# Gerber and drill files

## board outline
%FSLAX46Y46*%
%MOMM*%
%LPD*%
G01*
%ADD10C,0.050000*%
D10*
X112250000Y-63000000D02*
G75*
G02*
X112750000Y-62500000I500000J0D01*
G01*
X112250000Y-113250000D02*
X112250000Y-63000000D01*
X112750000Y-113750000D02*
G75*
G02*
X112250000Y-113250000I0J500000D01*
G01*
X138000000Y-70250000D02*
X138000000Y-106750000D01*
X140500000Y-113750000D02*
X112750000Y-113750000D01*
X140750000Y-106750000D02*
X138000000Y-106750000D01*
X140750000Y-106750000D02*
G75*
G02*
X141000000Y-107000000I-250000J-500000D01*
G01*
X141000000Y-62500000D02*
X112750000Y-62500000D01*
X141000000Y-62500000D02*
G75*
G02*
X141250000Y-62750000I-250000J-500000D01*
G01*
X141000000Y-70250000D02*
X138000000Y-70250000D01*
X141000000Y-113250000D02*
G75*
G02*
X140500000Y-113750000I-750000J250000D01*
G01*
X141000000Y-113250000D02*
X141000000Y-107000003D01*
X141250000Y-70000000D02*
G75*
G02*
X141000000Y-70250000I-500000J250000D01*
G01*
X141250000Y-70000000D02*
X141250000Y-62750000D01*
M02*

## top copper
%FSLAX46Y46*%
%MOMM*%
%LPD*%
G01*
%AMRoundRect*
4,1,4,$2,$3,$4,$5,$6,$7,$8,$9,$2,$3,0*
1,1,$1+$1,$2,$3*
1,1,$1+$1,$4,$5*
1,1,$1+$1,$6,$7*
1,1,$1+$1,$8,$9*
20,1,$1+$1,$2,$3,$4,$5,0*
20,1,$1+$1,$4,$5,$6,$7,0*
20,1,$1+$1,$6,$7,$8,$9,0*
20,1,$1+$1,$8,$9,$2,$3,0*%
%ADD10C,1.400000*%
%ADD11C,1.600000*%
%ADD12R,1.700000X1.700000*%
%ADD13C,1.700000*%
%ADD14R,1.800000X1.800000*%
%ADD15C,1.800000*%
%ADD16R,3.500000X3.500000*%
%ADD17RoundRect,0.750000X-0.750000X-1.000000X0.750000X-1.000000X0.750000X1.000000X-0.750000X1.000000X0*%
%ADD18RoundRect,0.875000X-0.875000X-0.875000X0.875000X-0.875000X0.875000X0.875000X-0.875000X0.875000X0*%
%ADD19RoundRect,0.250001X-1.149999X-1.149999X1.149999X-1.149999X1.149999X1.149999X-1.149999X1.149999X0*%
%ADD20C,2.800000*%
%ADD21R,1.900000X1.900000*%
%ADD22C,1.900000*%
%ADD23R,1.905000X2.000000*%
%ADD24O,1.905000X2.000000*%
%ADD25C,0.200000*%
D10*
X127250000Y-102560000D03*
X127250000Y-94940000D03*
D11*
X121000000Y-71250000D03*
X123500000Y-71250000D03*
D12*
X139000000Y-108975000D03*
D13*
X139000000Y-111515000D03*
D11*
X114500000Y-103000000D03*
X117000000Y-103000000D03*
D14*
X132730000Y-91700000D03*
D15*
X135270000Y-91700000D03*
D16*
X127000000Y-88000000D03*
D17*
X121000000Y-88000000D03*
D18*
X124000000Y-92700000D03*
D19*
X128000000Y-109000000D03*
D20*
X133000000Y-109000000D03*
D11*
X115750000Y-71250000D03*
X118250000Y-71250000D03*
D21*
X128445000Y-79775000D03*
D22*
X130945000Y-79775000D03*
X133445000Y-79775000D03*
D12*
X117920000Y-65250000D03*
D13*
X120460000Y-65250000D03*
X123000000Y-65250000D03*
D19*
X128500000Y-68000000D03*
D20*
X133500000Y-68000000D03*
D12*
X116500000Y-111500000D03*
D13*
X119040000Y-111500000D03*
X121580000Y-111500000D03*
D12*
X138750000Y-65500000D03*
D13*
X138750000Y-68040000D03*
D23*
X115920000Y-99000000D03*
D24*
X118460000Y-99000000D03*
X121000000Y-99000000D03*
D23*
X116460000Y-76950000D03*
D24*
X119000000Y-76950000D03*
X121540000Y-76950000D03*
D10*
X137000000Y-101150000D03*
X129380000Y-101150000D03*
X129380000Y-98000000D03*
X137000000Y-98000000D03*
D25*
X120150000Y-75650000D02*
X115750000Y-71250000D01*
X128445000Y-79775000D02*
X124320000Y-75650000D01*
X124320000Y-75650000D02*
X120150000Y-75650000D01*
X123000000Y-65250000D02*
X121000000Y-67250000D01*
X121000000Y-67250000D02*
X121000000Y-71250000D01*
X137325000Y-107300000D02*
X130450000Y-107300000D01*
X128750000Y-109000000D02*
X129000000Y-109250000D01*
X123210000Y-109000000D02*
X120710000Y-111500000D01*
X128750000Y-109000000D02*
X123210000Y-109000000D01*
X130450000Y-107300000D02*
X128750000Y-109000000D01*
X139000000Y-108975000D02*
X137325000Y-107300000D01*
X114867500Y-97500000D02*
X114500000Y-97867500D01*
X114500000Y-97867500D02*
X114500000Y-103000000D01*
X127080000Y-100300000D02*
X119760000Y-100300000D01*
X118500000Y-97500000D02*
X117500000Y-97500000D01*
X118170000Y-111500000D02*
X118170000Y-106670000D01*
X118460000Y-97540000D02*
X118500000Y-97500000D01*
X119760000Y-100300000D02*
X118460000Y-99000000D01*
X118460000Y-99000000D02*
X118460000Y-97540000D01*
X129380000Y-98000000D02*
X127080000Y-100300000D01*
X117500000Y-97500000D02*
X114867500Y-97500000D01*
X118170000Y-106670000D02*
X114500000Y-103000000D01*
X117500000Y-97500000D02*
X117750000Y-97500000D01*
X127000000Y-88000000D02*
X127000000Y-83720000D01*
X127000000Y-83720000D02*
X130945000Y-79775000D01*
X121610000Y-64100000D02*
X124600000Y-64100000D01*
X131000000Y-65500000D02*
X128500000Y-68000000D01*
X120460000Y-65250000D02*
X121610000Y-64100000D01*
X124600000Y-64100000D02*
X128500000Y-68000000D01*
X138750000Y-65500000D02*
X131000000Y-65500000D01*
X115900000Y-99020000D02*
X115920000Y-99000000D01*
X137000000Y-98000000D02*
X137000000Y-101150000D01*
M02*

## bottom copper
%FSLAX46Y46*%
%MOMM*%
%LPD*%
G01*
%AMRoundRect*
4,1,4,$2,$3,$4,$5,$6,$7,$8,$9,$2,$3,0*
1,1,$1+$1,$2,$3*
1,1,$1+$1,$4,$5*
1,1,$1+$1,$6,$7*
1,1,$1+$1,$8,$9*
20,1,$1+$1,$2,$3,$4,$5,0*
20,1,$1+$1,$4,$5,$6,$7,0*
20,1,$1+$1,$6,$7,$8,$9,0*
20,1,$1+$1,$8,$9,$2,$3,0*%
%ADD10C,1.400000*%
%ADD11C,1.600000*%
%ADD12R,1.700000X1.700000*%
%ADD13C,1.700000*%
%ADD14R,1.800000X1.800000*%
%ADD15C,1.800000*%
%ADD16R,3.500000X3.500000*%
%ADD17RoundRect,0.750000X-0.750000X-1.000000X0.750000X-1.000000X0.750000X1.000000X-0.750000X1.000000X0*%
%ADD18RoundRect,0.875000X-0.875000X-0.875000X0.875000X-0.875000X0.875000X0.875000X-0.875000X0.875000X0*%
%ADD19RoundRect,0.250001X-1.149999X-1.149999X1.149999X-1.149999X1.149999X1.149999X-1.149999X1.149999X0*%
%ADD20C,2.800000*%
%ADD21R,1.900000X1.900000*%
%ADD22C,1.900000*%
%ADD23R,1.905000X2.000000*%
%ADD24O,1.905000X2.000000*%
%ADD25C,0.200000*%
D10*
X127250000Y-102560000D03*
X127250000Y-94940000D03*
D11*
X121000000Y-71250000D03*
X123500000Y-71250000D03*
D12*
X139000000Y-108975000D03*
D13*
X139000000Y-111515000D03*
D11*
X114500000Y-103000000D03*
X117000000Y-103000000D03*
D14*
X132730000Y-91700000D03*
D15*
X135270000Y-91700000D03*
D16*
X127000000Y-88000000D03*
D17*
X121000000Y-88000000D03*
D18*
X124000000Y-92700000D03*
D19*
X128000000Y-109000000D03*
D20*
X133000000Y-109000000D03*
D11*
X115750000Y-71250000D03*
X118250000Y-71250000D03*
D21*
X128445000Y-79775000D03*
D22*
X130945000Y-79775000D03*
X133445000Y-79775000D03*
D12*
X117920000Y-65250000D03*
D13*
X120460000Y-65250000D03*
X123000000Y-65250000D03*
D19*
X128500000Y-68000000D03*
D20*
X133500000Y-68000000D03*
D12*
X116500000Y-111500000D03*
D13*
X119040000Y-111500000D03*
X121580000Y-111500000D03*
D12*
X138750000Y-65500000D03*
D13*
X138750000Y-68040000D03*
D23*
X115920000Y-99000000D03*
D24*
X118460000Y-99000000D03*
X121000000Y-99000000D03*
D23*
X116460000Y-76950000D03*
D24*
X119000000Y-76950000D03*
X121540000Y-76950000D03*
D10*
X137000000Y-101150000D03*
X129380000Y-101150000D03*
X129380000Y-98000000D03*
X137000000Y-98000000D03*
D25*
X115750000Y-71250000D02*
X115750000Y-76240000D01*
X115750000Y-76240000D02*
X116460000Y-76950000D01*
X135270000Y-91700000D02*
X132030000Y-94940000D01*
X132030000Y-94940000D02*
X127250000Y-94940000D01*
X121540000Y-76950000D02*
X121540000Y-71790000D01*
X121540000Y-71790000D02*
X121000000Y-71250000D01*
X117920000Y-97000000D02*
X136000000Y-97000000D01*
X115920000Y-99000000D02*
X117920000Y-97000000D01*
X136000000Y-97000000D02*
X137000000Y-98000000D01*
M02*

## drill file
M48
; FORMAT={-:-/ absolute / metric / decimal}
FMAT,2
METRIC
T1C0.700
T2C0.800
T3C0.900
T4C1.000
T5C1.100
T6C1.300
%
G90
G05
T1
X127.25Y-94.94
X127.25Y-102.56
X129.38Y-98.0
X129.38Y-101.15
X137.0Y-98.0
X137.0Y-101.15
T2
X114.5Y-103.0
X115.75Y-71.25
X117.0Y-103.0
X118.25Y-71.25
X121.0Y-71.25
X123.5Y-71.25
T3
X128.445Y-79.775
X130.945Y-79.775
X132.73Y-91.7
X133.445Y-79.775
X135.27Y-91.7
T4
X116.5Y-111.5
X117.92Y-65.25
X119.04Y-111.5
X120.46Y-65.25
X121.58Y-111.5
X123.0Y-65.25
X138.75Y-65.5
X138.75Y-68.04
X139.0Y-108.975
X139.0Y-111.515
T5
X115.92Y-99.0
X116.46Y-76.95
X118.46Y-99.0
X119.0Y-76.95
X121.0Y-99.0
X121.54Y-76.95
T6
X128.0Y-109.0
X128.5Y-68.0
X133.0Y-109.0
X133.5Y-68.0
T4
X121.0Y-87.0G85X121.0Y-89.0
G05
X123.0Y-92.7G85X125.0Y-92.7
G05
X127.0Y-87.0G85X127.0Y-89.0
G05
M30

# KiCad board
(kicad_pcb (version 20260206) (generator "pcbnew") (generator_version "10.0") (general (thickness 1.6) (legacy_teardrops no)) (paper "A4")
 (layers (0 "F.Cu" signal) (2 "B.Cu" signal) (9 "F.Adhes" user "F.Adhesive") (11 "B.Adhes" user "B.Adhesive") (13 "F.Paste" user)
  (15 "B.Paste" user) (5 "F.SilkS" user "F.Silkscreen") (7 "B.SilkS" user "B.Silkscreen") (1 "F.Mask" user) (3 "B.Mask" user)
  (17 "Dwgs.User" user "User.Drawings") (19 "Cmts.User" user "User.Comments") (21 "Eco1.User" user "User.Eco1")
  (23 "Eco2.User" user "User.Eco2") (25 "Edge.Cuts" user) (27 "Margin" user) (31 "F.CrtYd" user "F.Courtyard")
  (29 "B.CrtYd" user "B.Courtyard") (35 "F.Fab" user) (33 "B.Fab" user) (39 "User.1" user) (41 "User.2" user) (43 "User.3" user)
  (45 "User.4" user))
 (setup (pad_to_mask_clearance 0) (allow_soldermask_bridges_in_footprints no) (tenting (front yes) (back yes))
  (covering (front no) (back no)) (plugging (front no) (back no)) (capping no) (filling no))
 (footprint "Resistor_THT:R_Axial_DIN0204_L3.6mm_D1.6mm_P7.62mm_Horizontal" (layer "F.Cu") (at 127.25 102.56 90)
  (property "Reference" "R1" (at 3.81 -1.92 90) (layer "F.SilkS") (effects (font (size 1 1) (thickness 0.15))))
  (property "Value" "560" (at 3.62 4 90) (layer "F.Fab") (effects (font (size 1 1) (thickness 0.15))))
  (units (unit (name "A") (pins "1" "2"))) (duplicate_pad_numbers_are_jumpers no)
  (pad "1" thru_hole circle (at 0 0 90) (size 1.4 1.4) (drill 0.7) (layers "*.Cu" "*.Mask") (remove_unused_layers no) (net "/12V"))
  (pad "2" thru_hole circle (at 7.62 0 90) (size 1.4 1.4) (drill 0.7) (layers "*.Cu" "*.Mask") (remove_unused_layers no) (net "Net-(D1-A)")))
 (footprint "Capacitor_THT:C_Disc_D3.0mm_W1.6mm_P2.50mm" (layer "F.Cu") (at 121 71.25)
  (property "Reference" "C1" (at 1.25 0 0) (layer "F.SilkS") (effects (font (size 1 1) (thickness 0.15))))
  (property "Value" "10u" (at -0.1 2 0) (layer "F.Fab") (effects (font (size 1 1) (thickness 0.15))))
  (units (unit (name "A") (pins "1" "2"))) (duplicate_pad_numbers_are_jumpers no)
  (pad "1" thru_hole circle (at 0 0) (size 1.6 1.6) (drill 0.8) (layers "*.Cu" "*.Mask") (remove_unused_layers no) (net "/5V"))
  (pad "2" thru_hole circle (at 2.5 0) (size 1.6 1.6) (drill 0.8) (layers "*.Cu" "*.Mask") (remove_unused_layers no) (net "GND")))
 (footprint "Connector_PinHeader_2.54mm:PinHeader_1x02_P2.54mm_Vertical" (layer "F.Cu") (at 139 108.975)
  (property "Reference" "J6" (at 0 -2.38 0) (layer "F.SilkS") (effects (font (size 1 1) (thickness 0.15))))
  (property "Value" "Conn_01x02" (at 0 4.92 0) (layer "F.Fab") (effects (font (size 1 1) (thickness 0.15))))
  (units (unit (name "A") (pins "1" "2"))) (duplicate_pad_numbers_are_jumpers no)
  (pad "1" thru_hole rect (at 0 0) (size 1.7 1.7) (drill 1) (layers "*.Cu" "*.Mask") (remove_unused_layers no) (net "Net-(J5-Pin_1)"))
  (pad "2" thru_hole circle (at 0 2.54) (size 1.7 1.7) (drill 1) (layers "*.Cu" "*.Mask") (remove_unused_layers no) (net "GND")))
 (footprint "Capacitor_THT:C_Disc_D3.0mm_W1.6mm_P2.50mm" (layer "F.Cu") (at 114.5 103)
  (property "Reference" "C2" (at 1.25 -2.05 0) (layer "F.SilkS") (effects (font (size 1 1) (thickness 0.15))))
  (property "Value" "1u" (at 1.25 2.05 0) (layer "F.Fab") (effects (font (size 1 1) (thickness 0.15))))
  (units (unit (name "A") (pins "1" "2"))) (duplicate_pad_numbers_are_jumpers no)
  (pad "1" thru_hole circle (at 0 0) (size 1.6 1.6) (drill 0.8) (layers "*.Cu" "*.Mask") (remove_unused_layers no) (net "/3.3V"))
  (pad "2" thru_hole circle (at 2.5 0) (size 1.6 1.6) (drill 0.8) (layers "*.Cu" "*.Mask") (remove_unused_layers no) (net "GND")))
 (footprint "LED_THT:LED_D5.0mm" (layer "F.Cu") (at 132.73 91.7)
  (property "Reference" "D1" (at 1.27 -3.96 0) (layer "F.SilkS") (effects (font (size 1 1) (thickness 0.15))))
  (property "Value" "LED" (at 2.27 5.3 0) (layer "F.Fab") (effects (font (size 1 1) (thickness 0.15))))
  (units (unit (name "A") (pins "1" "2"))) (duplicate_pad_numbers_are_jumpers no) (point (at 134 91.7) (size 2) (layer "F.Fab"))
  (pad "1" thru_hole rect (at 0 0) (size 1.8 1.8) (drill 0.9) (layers "*.Cu" "*.Mask") (remove_unused_layers no) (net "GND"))
  (pad "2" thru_hole circle (at 2.54 0) (size 1.8 1.8) (drill 0.9) (layers "*.Cu" "*.Mask") (remove_unused_layers no) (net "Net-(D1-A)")))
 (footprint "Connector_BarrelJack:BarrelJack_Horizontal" (layer "F.Cu") (at 127 88)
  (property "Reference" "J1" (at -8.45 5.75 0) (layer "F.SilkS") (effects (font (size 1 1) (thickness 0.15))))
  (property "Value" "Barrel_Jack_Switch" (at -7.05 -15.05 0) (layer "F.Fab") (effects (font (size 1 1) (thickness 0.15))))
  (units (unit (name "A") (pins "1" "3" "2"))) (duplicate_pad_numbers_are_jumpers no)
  (pad "1" thru_hole rect (at 0 0) (size 3.5 3.5) (drill oval 1 3) (layers "*.Cu" "*.Mask") (remove_unused_layers no) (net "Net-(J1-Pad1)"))
  (pad "2" thru_hole roundrect (at -6 0) (size 3 3.5) (drill oval 1 3) (layers "*.Cu" "*.Mask") (remove_unused_layers no)
   (roundrect_rratio 0.25) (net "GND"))
  (pad "3" thru_hole roundrect (at -3 4.7) (size 3.5 3.5) (drill oval 3 1) (layers "*.Cu" "*.Mask") (remove_unused_layers no)
   (roundrect_rratio 0.25) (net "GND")))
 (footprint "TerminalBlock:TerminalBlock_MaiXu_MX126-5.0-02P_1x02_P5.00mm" (layer "F.Cu") (at 128 109)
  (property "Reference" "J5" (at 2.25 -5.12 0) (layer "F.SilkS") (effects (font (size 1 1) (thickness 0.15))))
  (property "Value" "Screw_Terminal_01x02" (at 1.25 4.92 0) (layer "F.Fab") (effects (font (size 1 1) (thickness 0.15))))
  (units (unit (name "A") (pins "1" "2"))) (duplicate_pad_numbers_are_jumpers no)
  (pad "1" thru_hole roundrect (at 0 0) (size 2.8 2.8) (drill 1.3) (layers "*.Cu" "*.Mask") (remove_unused_layers no)
   (roundrect_rratio 0.089286) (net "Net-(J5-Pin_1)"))
  (pad "2" thru_hole circle (at 5 0) (size 2.8 2.8) (drill 1.3) (layers "*.Cu" "*.Mask") (remove_unused_layers no) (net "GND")))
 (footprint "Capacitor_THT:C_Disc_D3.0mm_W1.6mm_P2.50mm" (layer "F.Cu") (at 115.75 71.25)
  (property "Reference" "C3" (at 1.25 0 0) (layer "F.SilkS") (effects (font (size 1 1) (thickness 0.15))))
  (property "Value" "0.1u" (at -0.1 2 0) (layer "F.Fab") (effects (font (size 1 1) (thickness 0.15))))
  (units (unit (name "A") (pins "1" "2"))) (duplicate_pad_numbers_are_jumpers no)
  (pad "1" thru_hole circle (at 0 0) (size 1.6 1.6) (drill 0.8) (layers "*.Cu" "*.Mask") (remove_unused_layers no) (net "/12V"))
  (pad "2" thru_hole circle (at 2.5 0) (size 1.6 1.6) (drill 0.8) (layers "*.Cu" "*.Mask") (remove_unused_layers no) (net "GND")))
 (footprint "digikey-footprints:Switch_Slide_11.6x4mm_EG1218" (layer "F.Cu") (at 128.445 79.775)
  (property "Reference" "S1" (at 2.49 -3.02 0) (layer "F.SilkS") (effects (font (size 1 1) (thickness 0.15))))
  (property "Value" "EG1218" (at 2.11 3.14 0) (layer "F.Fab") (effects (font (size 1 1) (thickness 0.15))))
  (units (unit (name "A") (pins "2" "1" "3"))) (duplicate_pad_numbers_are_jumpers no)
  (pad "1" thru_hole rect (at 0 0) (size 1.9 1.9) (drill 0.9) (layers "*.Cu" "*.Mask") (remove_unused_layers no) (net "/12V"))
  (pad "2" thru_hole circle (at 2.5 0) (size 1.9 1.9) (drill 0.9) (layers "*.Cu" "*.Mask") (remove_unused_layers no) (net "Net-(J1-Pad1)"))
  (pad "3" thru_hole circle (at 5 0) (size 1.9 1.9) (drill 0.9) (layers "*.Cu" "*.Mask") (remove_unused_layers no)
   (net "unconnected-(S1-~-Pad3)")))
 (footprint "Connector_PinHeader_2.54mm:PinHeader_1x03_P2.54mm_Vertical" (layer "F.Cu") (at 117.92 65.25 90)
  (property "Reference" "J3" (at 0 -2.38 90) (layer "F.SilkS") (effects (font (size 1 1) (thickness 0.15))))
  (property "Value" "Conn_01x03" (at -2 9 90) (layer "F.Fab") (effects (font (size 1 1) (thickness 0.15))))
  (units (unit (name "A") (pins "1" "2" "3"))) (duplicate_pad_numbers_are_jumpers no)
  (pad "1" thru_hole rect (at 0 0 90) (size 1.7 1.7) (drill 1) (layers "*.Cu" "*.Mask") (remove_unused_layers no) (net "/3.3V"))
  (pad "2" thru_hole circle (at 0 2.54 90) (size 1.7 1.7) (drill 1) (layers "*.Cu" "*.Mask") (remove_unused_layers no)
   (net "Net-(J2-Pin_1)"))
  (pad "3" thru_hole circle (at 0 5.08 90) (size 1.7 1.7) (drill 1) (layers "*.Cu" "*.Mask") (remove_unused_layers no) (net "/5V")))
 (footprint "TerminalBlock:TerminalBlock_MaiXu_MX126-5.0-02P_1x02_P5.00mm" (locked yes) (layer "F.Cu") (at 128.5 68)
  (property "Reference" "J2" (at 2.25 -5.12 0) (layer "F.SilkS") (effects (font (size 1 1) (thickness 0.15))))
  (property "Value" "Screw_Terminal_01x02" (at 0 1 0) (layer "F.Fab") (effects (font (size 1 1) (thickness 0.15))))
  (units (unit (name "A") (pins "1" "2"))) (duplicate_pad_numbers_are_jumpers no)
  (pad "1" thru_hole roundrect (at 0 0) (size 2.8 2.8) (drill 1.3) (layers "*.Cu" "*.Mask") (remove_unused_layers no)
   (roundrect_rratio 0.089286) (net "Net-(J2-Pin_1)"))
  (pad "2" thru_hole circle (at 5 0) (size 2.8 2.8) (drill 1.3) (layers "*.Cu" "*.Mask") (remove_unused_layers no) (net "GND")))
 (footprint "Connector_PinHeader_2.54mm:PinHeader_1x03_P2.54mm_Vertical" (layer "F.Cu") (at 116.5 111.5 90)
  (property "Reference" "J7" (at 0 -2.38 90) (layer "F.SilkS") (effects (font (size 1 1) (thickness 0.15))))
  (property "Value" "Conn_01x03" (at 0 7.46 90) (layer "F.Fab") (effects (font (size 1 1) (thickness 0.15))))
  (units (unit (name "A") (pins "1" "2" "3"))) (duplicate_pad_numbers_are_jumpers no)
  (pad "1" thru_hole rect (at 0 0 90) (size 1.7 1.7) (drill 1) (layers "*.Cu" "*.Mask") (remove_unused_layers no) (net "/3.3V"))
  (pad "2" thru_hole circle (at 0 2.54 90) (size 1.7 1.7) (drill 1) (layers "*.Cu" "*.Mask") (remove_unused_layers no)
   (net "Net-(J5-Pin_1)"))
  (pad "3" thru_hole circle (at 0 5.08 90) (size 1.7 1.7) (drill 1) (layers "*.Cu" "*.Mask") (remove_unused_layers no) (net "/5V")))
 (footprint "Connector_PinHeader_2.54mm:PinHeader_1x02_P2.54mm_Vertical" (layer "F.Cu") (at 138.75 65.5)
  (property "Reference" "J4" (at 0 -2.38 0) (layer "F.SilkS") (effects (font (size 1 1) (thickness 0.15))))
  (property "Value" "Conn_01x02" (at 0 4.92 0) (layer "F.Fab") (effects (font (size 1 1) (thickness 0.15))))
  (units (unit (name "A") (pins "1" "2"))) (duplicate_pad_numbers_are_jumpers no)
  (pad "1" thru_hole rect (at 0 0) (size 1.7 1.7) (drill 1) (layers "*.Cu" "*.Mask") (remove_unused_layers no) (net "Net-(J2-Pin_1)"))
  (pad "2" thru_hole circle (at 0 2.54) (size 1.7 1.7) (drill 1) (layers "*.Cu" "*.Mask") (remove_unused_layers no) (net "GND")))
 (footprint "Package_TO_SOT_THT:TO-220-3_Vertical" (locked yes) (layer "F.Cu") (at 115.92 99)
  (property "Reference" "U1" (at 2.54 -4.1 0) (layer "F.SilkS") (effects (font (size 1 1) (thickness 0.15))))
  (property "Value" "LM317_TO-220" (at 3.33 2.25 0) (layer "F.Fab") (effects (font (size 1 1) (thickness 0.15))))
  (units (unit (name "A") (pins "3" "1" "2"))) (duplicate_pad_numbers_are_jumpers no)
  (pad "1" thru_hole rect (at 0 0) (size 1.905 2) (drill 1.1) (layers "*.Cu" "*.Mask") (remove_unused_layers no) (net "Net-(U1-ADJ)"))
  (pad "2" thru_hole oval (at 2.54 0) (size 1.905 2) (drill 1.1) (layers "*.Cu" "*.Mask") (remove_unused_layers no) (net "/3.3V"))
  (pad "3" thru_hole oval (at 5.08 0) (size 1.905 2) (drill 1.1) (layers "*.Cu" "*.Mask") (remove_unused_layers no) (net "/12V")))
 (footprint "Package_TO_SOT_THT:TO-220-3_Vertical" (layer "F.Cu") (at 116.46 76.95)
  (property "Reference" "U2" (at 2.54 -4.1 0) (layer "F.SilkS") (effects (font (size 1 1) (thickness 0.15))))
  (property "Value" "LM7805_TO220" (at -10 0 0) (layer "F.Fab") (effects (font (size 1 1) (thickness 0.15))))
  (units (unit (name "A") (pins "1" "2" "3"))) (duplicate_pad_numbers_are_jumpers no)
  (pad "1" thru_hole rect (at 0 0) (size 1.905 2) (drill 1.1) (layers "*.Cu" "*.Mask") (remove_unused_layers no) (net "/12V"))
  (pad "2" thru_hole oval (at 2.54 0) (size 1.905 2) (drill 1.1) (layers "*.Cu" "*.Mask") (remove_unused_layers no) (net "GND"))
  (pad "3" thru_hole oval (at 5.08 0) (size 1.905 2) (drill 1.1) (layers "*.Cu" "*.Mask") (remove_unused_layers no) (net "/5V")))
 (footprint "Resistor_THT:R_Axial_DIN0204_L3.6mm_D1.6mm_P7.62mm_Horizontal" (layer "F.Cu") (at 137 101.15 180)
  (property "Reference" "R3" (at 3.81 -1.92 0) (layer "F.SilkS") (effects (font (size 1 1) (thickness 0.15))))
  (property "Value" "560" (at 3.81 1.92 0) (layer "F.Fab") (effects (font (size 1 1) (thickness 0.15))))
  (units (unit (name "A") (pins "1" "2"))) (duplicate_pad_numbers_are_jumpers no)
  (pad "1" thru_hole circle (at 0 0 180) (size 1.4 1.4) (drill 0.7) (layers "*.Cu" "*.Mask") (remove_unused_layers no) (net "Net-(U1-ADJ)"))
  (pad "2" thru_hole circle (at 7.62 0 180) (size 1.4 1.4) (drill 0.7) (layers "*.Cu" "*.Mask") (remove_unused_layers no) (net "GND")))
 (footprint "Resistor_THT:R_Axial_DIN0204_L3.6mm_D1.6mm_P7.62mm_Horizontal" (layer "F.Cu") (at 129.38 98)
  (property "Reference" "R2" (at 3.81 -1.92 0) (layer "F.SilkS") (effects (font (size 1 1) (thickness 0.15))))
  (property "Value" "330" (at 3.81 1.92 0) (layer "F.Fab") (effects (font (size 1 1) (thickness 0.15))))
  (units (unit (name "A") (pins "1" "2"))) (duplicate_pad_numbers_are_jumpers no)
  (pad "1" thru_hole circle (at 0 0) (size 1.4 1.4) (drill 0.7) (layers "*.Cu" "*.Mask") (remove_unused_layers no) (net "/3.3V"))
  (pad "2" thru_hole circle (at 7.62 0) (size 1.4 1.4) (drill 0.7) (layers "*.Cu" "*.Mask") (remove_unused_layers no) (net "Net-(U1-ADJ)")))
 (gr_arc (start 112.25 63) (mid 112.396447 62.646447) (end 112.75 62.5) (stroke (width 0.05) (type default)) (layer "Edge.Cuts"))
 (gr_line (start 112.25 113.25) (end 112.25 63) (stroke (width 0.05) (type default)) (layer "Edge.Cuts"))
 (gr_arc (start 112.75 113.75) (mid 112.396447 113.603553) (end 112.25 113.25) (stroke (width 0.05) (type default)) (layer "Edge.Cuts"))
 (gr_line (start 138 70.25) (end 138 106.75) (stroke (width 0.05) (type default)) (layer "Edge.Cuts"))
 (gr_line (start 140.5 113.75) (end 112.75 113.75) (stroke (width 0.05) (type default)) (layer "Edge.Cuts"))
 (gr_line (start 140.75 106.75) (end 138 106.75) (stroke (width 0.05) (type default)) (layer "Edge.Cuts"))
 (gr_arc (start 140.75 106.75) (mid 140.895285 106.854715) (end 141 107) (stroke (width 0.05) (type default)) (layer "Edge.Cuts"))
 (gr_line (start 141 62.5) (end 112.75 62.5) (stroke (width 0.05) (type default)) (layer "Edge.Cuts"))
 (gr_arc (start 141 62.5) (mid 141.145285 62.604715) (end 141.25 62.75) (stroke (width 0.05) (type default)) (layer "Edge.Cuts"))
 (gr_line (start 141 70.25) (end 138 70.25) (stroke (width 0.05) (type default)) (layer "Edge.Cuts"))
 (gr_arc (start 141 113.25) (mid 140.809017 113.559017) (end 140.5 113.75) (stroke (width 0.05) (type default)) (layer "Edge.Cuts"))
 (gr_line (start 141 113.25) (end 141 107.000003) (stroke (width 0.05) (type default)) (layer "Edge.Cuts"))
 (gr_arc (start 141.25 70) (mid 141.145285 70.145285) (end 141 70.25) (stroke (width 0.05) (type default)) (layer "Edge.Cuts"))
 (gr_line (start 141.25 70) (end 141.25 62.75) (stroke (width 0.05) (type default)) (layer "Edge.Cuts"))
 (segment (start 120.15 75.65) (end 115.75 71.25) (width 0.2) (layer "F.Cu") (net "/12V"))
 (segment (start 128.445 79.775) (end 124.32 75.65) (width 0.2) (layer "F.Cu") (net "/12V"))
 (segment (start 124.32 75.65) (end 120.15 75.65) (width 0.2) (layer "F.Cu") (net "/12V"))
 (segment (start 115.75 71.25) (end 115.75 76.24) (width 0.2) (layer "B.Cu") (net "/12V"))
 (segment (start 115.75 76.24) (end 116.46 76.95) (width 0.2) (layer "B.Cu") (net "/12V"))
 (segment (start 135.27 91.7) (end 132.03 94.94) (width 0.2) (layer "B.Cu") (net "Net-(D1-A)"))
 (segment (start 132.03 94.94) (end 127.25 94.94) (width 0.2) (layer "B.Cu") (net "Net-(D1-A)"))
 (segment (start 123 65.25) (end 121 67.25) (width 0.2) (layer "F.Cu") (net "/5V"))
 (segment (start 121 67.25) (end 121 71.25) (width 0.2) (layer "F.Cu") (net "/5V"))
 (segment (start 121.54 76.95) (end 121.54 71.79) (width 0.2) (layer "B.Cu") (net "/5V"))
 (segment (start 121.54 71.79) (end 121 71.25) (width 0.2) (layer "B.Cu") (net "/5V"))
 (segment (start 137.325 107.3) (end 130.45 107.3) (width 0.2) (layer "F.Cu") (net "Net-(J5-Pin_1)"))
 (segment (start 128.75 109) (end 129 109.25) (width 0.2) (layer "F.Cu") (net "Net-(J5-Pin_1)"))
 (segment (start 123.21 109) (end 120.71 111.5) (width 0.2) (layer "F.Cu") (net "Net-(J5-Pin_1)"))
 (segment (start 128.75 109) (end 123.21 109) (width 0.2) (layer "F.Cu") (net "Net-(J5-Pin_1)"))
 (segment (start 130.45 107.3) (end 128.75 109) (width 0.2) (layer "F.Cu") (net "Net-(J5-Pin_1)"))
 (segment (start 139 108.975) (end 137.325 107.3) (width 0.2) (layer "F.Cu") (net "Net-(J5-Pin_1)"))
 (segment (start 114.8675 97.5) (end 114.5 97.8675) (width 0.2) (layer "F.Cu") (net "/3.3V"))
 (segment (start 114.5 97.8675) (end 114.5 103) (width 0.2) (layer "F.Cu") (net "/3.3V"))
 (segment (start 127.08 100.3) (end 119.76 100.3) (width 0.2) (layer "F.Cu") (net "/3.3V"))
 (segment (start 118.5 97.5) (end 117.5 97.5) (width 0.2) (layer "F.Cu") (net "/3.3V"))
 (segment (start 118.17 111.5) (end 118.17 106.67) (width 0.2) (layer "F.Cu") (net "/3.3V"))
 (segment (start 118.46 97.54) (end 118.5 97.5) (width 0.2) (layer "F.Cu") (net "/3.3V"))
 (segment (start 119.76 100.3) (end 118.46 99) (width 0.2) (layer "F.Cu") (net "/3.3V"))
 (segment (start 118.46 99) (end 118.46 97.54) (width 0.2) (layer "F.Cu") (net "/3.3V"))
 (segment (start 129.38 98) (end 127.08 100.3) (width 0.2) (layer "F.Cu") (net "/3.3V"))
 (segment (start 117.5 97.5) (end 114.8675 97.5) (width 0.2) (layer "F.Cu") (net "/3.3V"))
 (segment (start 118.17 106.67) (end 114.5 103) (width 0.2) (layer "F.Cu") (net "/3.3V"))
 (segment (start 117.5 97.5) (end 117.75 97.5) (width 0.2) (layer "F.Cu") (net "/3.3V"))
 (segment (start 127 88) (end 127 83.72) (width 0.2) (layer "F.Cu") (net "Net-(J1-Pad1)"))
 (segment (start 127 83.72) (end 130.945 79.775) (width 0.2) (layer "F.Cu") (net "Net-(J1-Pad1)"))
 (segment (start 121.61 64.1) (end 124.6 64.1) (width 0.2) (layer "F.Cu") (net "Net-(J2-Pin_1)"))
 (segment (start 131 65.5) (end 128.5 68) (width 0.2) (layer "F.Cu") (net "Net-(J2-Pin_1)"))
 (segment (start 120.46 65.25) (end 121.61 64.1) (width 0.2) (layer "F.Cu") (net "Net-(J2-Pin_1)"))
 (segment (start 124.6 64.1) (end 128.5 68) (width 0.2) (layer "F.Cu") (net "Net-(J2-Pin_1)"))
 (segment (start 138.75 65.5) (end 131 65.5) (width 0.2) (layer "F.Cu") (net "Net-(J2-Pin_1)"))
 (segment (start 115.9 99.02) (end 115.92 99) (width 0.2) (layer "F.Cu") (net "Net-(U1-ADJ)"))
 (segment (start 137 98) (end 137 101.15) (width 0.2) (layer "F.Cu") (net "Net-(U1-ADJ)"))
 (segment (start 117.92 97) (end 136 97) (width 0.2) (layer "B.Cu") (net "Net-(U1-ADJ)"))
 (segment (start 115.92 99) (end 117.92 97) (width 0.2) (layer "B.Cu") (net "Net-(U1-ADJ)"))
 (segment (start 136 97) (end 137 98) (width 0.2) (layer "B.Cu") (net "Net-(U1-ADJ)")))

